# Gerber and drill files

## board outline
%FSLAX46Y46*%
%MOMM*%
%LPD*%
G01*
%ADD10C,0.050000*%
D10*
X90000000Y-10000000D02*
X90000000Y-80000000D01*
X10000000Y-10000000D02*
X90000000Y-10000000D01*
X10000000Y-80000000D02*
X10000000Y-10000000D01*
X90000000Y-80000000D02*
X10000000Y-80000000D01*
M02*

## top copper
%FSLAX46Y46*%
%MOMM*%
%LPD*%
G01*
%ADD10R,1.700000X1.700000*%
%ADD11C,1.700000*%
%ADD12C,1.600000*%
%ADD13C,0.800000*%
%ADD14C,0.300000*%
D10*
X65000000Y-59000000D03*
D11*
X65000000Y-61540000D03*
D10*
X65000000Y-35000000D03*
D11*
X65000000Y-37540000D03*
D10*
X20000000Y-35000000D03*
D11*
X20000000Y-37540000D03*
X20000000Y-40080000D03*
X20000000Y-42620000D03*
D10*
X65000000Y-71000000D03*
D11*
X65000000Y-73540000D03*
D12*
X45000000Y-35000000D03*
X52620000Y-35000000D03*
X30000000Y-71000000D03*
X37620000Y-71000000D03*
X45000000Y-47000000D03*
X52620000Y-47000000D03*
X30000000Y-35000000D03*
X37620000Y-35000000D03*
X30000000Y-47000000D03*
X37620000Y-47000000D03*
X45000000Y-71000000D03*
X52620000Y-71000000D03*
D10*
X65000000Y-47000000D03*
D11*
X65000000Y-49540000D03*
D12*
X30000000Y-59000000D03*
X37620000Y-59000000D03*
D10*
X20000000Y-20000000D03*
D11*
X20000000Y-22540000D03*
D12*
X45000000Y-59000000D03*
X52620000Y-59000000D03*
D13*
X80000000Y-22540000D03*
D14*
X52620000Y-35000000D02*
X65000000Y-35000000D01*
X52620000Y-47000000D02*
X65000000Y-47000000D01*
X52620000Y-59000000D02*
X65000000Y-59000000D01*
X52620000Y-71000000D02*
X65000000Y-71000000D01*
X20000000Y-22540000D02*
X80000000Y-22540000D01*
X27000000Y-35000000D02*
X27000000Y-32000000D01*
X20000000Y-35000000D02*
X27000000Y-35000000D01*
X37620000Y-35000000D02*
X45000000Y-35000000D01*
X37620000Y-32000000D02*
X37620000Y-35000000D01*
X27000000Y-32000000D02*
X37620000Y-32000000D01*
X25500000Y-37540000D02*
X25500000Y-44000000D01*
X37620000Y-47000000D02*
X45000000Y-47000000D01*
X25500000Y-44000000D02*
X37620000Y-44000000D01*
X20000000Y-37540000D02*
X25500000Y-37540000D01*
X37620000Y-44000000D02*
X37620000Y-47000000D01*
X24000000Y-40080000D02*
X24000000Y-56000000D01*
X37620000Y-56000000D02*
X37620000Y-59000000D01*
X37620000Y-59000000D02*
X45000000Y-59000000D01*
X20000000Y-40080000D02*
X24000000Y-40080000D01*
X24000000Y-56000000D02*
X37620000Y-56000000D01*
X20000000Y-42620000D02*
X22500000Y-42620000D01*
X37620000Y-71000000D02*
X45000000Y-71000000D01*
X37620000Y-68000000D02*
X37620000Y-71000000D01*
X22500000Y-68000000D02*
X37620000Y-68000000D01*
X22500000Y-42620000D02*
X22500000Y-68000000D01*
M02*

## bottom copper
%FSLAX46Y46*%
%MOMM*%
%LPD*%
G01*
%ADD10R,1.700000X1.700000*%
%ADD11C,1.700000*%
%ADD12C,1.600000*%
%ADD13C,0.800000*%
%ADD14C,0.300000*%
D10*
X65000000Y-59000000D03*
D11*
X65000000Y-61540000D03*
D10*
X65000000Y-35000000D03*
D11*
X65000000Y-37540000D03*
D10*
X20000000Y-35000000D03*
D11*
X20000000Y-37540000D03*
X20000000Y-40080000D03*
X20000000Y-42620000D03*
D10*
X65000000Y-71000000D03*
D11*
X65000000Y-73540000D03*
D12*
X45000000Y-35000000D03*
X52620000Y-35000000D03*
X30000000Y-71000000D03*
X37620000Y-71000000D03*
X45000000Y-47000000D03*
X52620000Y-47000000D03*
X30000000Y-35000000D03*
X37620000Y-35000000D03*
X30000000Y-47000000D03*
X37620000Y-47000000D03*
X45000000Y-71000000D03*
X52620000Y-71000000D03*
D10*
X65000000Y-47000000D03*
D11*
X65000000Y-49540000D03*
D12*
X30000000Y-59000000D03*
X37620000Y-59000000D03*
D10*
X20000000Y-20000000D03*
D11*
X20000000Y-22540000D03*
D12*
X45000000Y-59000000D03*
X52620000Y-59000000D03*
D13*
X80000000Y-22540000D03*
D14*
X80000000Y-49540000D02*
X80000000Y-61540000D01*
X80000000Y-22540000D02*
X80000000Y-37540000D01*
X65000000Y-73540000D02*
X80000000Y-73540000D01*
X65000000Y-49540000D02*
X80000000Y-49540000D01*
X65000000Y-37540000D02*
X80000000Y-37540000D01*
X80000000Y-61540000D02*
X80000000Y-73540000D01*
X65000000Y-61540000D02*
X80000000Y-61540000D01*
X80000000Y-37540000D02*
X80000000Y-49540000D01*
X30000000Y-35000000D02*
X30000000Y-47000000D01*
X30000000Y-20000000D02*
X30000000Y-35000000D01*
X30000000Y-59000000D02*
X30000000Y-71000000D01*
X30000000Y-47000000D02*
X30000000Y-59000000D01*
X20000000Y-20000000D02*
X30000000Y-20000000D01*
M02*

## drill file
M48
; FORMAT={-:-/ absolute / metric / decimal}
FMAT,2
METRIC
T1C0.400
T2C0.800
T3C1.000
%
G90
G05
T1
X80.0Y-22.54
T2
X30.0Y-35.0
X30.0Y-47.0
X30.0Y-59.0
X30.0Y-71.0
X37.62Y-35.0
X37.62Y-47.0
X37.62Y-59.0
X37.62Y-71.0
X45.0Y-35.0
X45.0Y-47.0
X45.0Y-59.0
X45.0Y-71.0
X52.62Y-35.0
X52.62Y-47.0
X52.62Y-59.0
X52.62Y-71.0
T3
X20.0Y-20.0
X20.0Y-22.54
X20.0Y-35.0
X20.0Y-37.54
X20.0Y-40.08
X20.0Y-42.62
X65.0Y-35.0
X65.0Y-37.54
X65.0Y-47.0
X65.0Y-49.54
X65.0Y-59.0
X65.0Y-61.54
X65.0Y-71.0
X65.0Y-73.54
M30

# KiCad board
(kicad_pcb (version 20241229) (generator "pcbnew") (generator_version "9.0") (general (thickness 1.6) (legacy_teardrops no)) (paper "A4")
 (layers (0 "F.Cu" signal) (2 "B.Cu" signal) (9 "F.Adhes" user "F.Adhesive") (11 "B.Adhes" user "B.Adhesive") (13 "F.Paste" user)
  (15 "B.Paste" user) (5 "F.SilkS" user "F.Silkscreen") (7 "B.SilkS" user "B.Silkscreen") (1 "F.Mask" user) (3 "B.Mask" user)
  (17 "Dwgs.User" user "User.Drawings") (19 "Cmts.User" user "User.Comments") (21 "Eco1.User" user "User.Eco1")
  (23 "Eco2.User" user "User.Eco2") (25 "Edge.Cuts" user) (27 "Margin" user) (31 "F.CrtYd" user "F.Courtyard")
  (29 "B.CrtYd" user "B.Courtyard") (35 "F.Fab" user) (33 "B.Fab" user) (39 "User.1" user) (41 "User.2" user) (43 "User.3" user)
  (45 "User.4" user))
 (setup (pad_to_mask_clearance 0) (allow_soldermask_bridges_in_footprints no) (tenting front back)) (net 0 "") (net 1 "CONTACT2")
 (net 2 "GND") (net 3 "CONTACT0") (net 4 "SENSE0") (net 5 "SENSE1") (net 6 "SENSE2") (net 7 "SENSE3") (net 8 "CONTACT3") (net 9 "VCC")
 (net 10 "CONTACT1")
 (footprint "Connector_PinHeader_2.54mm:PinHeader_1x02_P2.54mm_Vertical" (layer "F.Cu") (at 65 59)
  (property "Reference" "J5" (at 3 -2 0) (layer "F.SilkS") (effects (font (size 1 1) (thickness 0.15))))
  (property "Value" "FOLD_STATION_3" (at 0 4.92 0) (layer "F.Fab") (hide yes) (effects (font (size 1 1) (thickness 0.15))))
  (pad "1" thru_hole rect (at 0 0) (size 1.7 1.7) (drill 1) (layers "*.Cu" "*.Mask") (remove_unused_layers no) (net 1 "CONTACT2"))
  (pad "2" thru_hole circle (at 0 2.54) (size 1.7 1.7) (drill 1) (layers "*.Cu" "*.Mask") (remove_unused_layers no) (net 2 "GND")))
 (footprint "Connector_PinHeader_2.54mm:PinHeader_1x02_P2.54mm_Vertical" (layer "F.Cu") (at 65 35)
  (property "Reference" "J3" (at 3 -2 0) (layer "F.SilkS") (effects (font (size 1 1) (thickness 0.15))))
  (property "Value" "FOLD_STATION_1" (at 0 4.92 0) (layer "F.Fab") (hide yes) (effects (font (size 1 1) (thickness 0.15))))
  (pad "1" thru_hole rect (at 0 0) (size 1.7 1.7) (drill 1) (layers "*.Cu" "*.Mask") (remove_unused_layers no) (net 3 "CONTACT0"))
  (pad "2" thru_hole circle (at 0 2.54) (size 1.7 1.7) (drill 1) (layers "*.Cu" "*.Mask") (remove_unused_layers no) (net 2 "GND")))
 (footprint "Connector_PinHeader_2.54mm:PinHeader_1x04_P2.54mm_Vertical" (layer "F.Cu") (at 20 35)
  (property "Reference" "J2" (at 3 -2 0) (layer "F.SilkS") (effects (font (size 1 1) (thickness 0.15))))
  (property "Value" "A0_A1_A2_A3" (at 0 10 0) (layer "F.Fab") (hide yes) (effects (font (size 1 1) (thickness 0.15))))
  (pad "1" thru_hole rect (at 0 0) (size 1.7 1.7) (drill 1) (layers "*.Cu" "*.Mask") (remove_unused_layers no) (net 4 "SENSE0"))
  (pad "2" thru_hole circle (at 0 2.54) (size 1.7 1.7) (drill 1) (layers "*.Cu" "*.Mask") (remove_unused_layers no) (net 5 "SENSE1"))
  (pad "3" thru_hole circle (at 0 5.08) (size 1.7 1.7) (drill 1) (layers "*.Cu" "*.Mask") (remove_unused_layers no) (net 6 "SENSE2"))
  (pad "4" thru_hole circle (at 0 7.62) (size 1.7 1.7) (drill 1) (layers "*.Cu" "*.Mask") (remove_unused_layers no) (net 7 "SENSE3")))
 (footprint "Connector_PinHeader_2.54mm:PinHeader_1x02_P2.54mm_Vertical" (layer "F.Cu") (at 65 71)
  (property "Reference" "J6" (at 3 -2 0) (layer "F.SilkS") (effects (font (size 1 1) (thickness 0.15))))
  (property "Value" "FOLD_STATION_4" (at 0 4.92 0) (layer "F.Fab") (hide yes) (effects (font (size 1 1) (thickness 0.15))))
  (pad "1" thru_hole rect (at 0 0) (size 1.7 1.7) (drill 1) (layers "*.Cu" "*.Mask") (remove_unused_layers no) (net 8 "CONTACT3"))
  (pad "2" thru_hole circle (at 0 2.54) (size 1.7 1.7) (drill 1) (layers "*.Cu" "*.Mask") (remove_unused_layers no) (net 2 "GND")))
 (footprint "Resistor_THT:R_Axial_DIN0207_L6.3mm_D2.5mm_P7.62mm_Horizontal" (layer "F.Cu") (at 45 35)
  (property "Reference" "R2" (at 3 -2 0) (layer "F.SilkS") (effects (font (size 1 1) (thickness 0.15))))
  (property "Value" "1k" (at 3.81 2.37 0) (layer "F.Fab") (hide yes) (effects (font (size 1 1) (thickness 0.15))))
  (pad "1" thru_hole circle (at 0 0) (size 1.6 1.6) (drill 0.8) (layers "*.Cu" "*.Mask") (remove_unused_layers no) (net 4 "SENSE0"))
  (pad "2" thru_hole circle (at 7.62 0) (size 1.6 1.6) (drill 0.8) (layers "*.Cu" "*.Mask") (remove_unused_layers no) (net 3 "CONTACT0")))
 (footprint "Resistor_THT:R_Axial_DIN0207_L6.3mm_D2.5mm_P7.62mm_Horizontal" (layer "F.Cu") (at 30 71)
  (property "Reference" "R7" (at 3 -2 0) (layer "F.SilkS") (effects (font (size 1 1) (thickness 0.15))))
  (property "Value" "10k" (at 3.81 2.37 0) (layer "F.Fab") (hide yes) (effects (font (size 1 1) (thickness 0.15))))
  (pad "1" thru_hole circle (at 0 0) (size 1.6 1.6) (drill 0.8) (layers "*.Cu" "*.Mask") (remove_unused_layers no) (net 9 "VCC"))
  (pad "2" thru_hole circle (at 7.62 0) (size 1.6 1.6) (drill 0.8) (layers "*.Cu" "*.Mask") (remove_unused_layers no) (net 7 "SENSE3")))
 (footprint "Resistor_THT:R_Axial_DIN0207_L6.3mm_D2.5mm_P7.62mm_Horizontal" (layer "F.Cu") (at 45 47)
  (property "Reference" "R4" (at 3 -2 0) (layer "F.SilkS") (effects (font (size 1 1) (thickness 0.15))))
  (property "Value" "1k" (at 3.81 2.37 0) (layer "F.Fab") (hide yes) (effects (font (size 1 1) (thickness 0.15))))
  (pad "1" thru_hole circle (at 0 0) (size 1.6 1.6) (drill 0.8) (layers "*.Cu" "*.Mask") (remove_unused_layers no) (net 5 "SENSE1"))
  (pad "2" thru_hole circle (at 7.62 0) (size 1.6 1.6) (drill 0.8) (layers "*.Cu" "*.Mask") (remove_unused_layers no) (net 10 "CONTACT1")))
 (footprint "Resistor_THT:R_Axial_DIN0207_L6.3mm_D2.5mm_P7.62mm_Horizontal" (layer "F.Cu") (at 30 35)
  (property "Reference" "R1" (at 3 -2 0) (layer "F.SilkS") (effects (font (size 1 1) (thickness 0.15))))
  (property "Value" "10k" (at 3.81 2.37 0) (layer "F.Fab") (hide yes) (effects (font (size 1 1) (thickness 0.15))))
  (pad "1" thru_hole circle (at 0 0) (size 1.6 1.6) (drill 0.8) (layers "*.Cu" "*.Mask") (remove_unused_layers no) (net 9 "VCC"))
  (pad "2" thru_hole circle (at 7.62 0) (size 1.6 1.6) (drill 0.8) (layers "*.Cu" "*.Mask") (remove_unused_layers no) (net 4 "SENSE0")))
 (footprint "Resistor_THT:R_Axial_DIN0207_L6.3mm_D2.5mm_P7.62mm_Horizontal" (layer "F.Cu") (at 30 47)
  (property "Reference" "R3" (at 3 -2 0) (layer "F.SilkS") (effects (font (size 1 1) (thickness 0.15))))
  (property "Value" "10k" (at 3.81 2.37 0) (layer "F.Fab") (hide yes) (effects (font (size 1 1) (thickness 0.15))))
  (pad "1" thru_hole circle (at 0 0) (size 1.6 1.6) (drill 0.8) (layers "*.Cu" "*.Mask") (remove_unused_layers no) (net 9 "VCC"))
  (pad "2" thru_hole circle (at 7.62 0) (size 1.6 1.6) (drill 0.8) (layers "*.Cu" "*.Mask") (remove_unused_layers no) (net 5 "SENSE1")))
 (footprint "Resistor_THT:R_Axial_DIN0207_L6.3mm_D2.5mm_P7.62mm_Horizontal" (layer "F.Cu") (at 45 71)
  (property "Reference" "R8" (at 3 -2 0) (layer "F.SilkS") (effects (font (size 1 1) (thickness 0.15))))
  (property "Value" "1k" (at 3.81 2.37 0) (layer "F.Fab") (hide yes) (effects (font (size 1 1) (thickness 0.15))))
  (pad "1" thru_hole circle (at 0 0) (size 1.6 1.6) (drill 0.8) (layers "*.Cu" "*.Mask") (remove_unused_layers no) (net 7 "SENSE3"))
  (pad "2" thru_hole circle (at 7.62 0) (size 1.6 1.6) (drill 0.8) (layers "*.Cu" "*.Mask") (remove_unused_layers no) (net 8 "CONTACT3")))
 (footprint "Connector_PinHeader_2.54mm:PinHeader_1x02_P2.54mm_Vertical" (layer "F.Cu") (at 65 47)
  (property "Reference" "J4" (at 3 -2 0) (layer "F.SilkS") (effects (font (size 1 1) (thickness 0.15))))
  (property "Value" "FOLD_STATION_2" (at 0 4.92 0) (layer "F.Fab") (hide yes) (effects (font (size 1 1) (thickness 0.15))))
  (pad "1" thru_hole rect (at 0 0) (size 1.7 1.7) (drill 1) (layers "*.Cu" "*.Mask") (remove_unused_layers no) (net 10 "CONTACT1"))
  (pad "2" thru_hole circle (at 0 2.54) (size 1.7 1.7) (drill 1) (layers "*.Cu" "*.Mask") (remove_unused_layers no) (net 2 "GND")))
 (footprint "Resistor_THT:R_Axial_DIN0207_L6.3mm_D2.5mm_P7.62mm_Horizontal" (layer "F.Cu") (at 30 59)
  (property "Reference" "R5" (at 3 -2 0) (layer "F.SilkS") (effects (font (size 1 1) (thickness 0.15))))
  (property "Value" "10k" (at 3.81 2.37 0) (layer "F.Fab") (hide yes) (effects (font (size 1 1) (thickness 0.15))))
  (pad "1" thru_hole circle (at 0 0) (size 1.6 1.6) (drill 0.8) (layers "*.Cu" "*.Mask") (remove_unused_layers no) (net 9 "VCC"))
  (pad "2" thru_hole circle (at 7.62 0) (size 1.6 1.6) (drill 0.8) (layers "*.Cu" "*.Mask") (remove_unused_layers no) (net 6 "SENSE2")))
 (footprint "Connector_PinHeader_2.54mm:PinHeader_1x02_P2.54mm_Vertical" (layer "F.Cu") (at 20 20)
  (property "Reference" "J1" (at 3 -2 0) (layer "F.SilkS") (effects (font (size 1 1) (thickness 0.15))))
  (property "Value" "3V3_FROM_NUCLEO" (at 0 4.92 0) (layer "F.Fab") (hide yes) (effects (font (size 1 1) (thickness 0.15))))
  (pad "1" thru_hole rect (at 0 0) (size 1.7 1.7) (drill 1) (layers "*.Cu" "*.Mask") (remove_unused_layers no) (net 9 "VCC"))
  (pad "2" thru_hole circle (at 0 2.54) (size 1.7 1.7) (drill 1) (layers "*.Cu" "*.Mask") (remove_unused_layers no) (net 2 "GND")))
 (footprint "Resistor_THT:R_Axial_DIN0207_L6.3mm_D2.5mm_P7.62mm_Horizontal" (layer "F.Cu") (at 45 59)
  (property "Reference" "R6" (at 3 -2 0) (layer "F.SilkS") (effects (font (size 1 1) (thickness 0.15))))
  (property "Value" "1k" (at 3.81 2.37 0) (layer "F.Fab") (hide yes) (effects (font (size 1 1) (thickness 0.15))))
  (pad "1" thru_hole circle (at 0 0) (size 1.6 1.6) (drill 0.8) (layers "*.Cu" "*.Mask") (remove_unused_layers no) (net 6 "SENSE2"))
  (pad "2" thru_hole circle (at 7.62 0) (size 1.6 1.6) (drill 0.8) (layers "*.Cu" "*.Mask") (remove_unused_layers no) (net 1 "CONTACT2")))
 (gr_line (start 90 10) (end 90 80) (stroke (width 0.05) (type default)) (layer "Edge.Cuts"))
 (gr_line (start 10 10) (end 90 10) (stroke (width 0.05) (type default)) (layer "Edge.Cuts"))
 (gr_line (start 10 80) (end 10 10) (stroke (width 0.05) (type default)) (layer "Edge.Cuts"))
 (gr_line (start 90 80) (end 10 80) (stroke (width 0.05) (type default)) (layer "Edge.Cuts"))
 (segment (start 52.62 35) (end 65 35) (width 0.3) (layer "F.Cu") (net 3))
 (segment (start 52.62 47) (end 65 47) (width 0.3) (layer "F.Cu") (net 10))
 (segment (start 52.62 59) (end 65 59) (width 0.3) (layer "F.Cu") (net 1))
 (segment (start 52.62 71) (end 65 71) (width 0.3) (layer "F.Cu") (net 8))
 (segment (start 20 22.54) (end 80 22.54) (width 0.3) (layer "F.Cu") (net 2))
 (via (at 80 22.54) (size 0.8) (drill 0.4) (layers "F.Cu" "B.Cu") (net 2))
 (segment (start 80 49.54) (end 80 61.54) (width 0.3) (layer "B.Cu") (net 2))
 (segment (start 80 22.54) (end 80 37.54) (width 0.3) (layer "B.Cu") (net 2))
 (segment (start 65 73.54) (end 80 73.54) (width 0.3) (layer "B.Cu") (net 2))
 (segment (start 65 49.54) (end 80 49.54) (width 0.3) (layer "B.Cu") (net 2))
 (segment (start 65 37.54) (end 80 37.54) (width 0.3) (layer "B.Cu") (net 2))
 (segment (start 80 61.54) (end 80 73.54) (width 0.3) (layer "B.Cu") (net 2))
 (segment (start 65 61.54) (end 80 61.54) (width 0.3) (layer "B.Cu") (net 2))
 (segment (start 80 37.54) (end 80 49.54) (width 0.3) (layer "B.Cu") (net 2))
 (segment (start 27 35) (end 27 32) (width 0.3) (layer "F.Cu") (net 4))
 (segment (start 20 35) (end 27 35) (width 0.3) (layer "F.Cu") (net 4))
 (segment (start 37.62 35) (end 45 35) (width 0.3) (layer "F.Cu") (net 4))
 (segment (start 37.62 32) (end 37.62 35) (width 0.3) (layer "F.Cu") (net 4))
 (segment (start 27 32) (end 37.62 32) (width 0.3) (layer "F.Cu") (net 4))
 (segment (start 25.5 37.54) (end 25.5 44) (width 0.3) (layer "F.Cu") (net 5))
 (segment (start 37.62 47) (end 45 47) (width 0.3) (layer "F.Cu") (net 5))
 (segment (start 25.5 44) (end 37.62 44) (width 0.3) (layer "F.Cu") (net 5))
 (segment (start 20 37.54) (end 25.5 37.54) (width 0.3) (layer "F.Cu") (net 5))
 (segment (start 37.62 44) (end 37.62 47) (width 0.3) (layer "F.Cu") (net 5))
 (segment (start 24 40.08) (end 24 56) (width 0.3) (layer "F.Cu") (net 6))
 (segment (start 37.62 56) (end 37.62 59) (width 0.3) (layer "F.Cu") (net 6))
 (segment (start 37.62 59) (end 45 59) (width 0.3) (layer "F.Cu") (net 6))
 (segment (start 20 40.08) (end 24 40.08) (width 0.3) (layer "F.Cu") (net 6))
 (segment (start 24 56) (end 37.62 56) (width 0.3) (layer "F.Cu") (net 6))
 (segment (start 20 42.62) (end 22.5 42.62) (width 0.3) (layer "F.Cu") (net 7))
 (segment (start 37.62 71) (end 45 71) (width 0.3) (layer "F.Cu") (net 7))
 (segment (start 37.62 68) (end 37.62 71) (width 0.3) (layer "F.Cu") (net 7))
 (segment (start 22.5 68) (end 37.62 68) (width 0.3) (layer "F.Cu") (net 7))
 (segment (start 22.5 42.62) (end 22.5 68) (width 0.3) (layer "F.Cu") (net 7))
 (segment (start 30 35) (end 30 47) (width 0.3) (layer "B.Cu") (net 9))
 (segment (start 30 20) (end 30 35) (width 0.3) (layer "B.Cu") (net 9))
 (segment (start 30 59) (end 30 71) (width 0.3) (layer "B.Cu") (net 9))
 (segment (start 30 47) (end 30 59) (width 0.3) (layer "B.Cu") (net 9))
 (segment (start 20 20) (end 30 20) (width 0.3) (layer "B.Cu") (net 9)))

